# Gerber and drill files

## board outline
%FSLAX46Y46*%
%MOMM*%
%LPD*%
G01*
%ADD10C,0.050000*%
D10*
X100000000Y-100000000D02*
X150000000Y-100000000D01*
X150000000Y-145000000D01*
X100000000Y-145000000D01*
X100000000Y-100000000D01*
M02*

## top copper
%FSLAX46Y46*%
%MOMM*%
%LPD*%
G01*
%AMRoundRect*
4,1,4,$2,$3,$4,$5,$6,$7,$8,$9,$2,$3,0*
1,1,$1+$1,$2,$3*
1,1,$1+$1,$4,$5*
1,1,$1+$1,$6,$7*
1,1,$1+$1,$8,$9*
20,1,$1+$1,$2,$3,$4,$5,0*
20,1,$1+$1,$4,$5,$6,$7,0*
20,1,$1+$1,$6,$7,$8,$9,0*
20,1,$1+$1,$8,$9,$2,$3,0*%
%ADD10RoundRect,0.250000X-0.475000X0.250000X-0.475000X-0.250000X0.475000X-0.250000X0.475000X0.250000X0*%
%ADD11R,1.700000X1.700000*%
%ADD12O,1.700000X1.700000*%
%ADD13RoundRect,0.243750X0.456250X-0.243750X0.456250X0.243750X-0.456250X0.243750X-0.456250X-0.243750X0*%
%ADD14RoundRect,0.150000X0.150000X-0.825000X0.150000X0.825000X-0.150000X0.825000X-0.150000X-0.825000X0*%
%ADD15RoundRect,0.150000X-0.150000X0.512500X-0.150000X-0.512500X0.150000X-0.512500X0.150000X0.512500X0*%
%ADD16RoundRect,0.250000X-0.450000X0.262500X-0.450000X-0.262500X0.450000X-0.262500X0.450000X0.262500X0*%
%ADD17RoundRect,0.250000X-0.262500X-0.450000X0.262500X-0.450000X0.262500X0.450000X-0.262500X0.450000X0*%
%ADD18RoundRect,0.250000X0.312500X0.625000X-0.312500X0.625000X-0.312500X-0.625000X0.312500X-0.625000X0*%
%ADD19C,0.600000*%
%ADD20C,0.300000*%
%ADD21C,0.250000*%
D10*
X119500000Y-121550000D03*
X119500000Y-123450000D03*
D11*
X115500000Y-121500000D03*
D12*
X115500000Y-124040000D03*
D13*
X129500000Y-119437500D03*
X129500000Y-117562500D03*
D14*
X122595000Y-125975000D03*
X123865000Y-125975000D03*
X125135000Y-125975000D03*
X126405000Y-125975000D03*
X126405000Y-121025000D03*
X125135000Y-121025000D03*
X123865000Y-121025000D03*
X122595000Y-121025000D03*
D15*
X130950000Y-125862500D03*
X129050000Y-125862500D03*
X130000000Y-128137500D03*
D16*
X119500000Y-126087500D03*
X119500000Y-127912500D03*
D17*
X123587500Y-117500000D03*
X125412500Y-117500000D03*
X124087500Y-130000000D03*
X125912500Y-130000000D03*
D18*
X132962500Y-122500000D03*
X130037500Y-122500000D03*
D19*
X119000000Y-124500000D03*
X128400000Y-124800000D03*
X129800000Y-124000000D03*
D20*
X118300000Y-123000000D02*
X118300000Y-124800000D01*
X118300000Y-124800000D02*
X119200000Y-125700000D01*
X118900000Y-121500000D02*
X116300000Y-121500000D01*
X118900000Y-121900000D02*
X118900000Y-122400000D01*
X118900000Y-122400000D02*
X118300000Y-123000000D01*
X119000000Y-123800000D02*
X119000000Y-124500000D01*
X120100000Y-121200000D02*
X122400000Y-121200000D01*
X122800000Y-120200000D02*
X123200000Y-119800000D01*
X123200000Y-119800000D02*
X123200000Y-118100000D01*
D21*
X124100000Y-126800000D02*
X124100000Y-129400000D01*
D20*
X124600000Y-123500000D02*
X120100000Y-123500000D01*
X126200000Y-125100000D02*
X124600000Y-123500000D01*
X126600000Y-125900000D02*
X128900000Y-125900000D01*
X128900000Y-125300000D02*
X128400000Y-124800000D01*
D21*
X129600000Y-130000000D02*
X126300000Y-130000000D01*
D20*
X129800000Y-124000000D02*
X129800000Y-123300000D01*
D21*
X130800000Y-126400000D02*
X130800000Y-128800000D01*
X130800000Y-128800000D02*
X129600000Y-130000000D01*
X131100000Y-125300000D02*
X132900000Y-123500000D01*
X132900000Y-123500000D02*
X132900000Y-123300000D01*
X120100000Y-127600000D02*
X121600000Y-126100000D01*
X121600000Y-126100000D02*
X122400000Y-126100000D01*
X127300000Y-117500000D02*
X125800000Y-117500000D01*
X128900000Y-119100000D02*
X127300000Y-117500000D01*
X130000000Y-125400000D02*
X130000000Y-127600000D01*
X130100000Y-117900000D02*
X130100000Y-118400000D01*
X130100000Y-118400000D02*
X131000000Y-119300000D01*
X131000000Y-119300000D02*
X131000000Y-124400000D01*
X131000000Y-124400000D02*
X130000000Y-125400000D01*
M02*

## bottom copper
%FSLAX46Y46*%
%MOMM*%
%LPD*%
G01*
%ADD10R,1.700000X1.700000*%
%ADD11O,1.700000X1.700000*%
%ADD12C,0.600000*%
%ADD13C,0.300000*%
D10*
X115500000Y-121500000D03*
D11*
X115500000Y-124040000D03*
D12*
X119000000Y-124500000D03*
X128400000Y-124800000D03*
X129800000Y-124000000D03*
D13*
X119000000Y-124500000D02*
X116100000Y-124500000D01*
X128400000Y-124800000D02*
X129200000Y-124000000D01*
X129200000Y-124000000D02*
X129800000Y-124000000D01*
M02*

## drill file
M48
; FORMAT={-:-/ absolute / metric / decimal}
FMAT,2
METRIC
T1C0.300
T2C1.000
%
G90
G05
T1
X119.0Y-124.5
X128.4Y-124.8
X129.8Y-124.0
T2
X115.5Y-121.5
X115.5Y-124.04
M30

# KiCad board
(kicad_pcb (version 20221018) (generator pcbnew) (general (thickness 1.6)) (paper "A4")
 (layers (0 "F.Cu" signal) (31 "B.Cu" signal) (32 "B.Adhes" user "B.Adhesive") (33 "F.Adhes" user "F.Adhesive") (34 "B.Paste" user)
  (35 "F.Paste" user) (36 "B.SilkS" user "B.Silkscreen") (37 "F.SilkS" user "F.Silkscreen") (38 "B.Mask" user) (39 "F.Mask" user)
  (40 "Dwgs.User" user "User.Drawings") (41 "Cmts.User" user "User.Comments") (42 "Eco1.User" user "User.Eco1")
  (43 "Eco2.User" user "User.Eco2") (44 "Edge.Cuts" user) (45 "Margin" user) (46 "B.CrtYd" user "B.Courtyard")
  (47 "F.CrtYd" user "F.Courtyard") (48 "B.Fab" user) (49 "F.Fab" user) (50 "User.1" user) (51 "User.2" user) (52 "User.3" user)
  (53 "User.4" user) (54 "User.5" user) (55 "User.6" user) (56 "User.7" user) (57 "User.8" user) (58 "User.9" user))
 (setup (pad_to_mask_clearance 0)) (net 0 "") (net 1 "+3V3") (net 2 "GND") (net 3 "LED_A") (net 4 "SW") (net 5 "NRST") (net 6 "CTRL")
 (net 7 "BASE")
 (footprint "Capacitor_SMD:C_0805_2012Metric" (layer "F.Cu") (at 119.5 122.5 -90)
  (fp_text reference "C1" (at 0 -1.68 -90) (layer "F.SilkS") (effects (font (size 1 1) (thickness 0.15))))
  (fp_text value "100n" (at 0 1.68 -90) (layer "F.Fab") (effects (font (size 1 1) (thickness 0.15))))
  (pad "1" smd roundrect (at -0.95 0 270) (size 1 1.45) (layers "F.Cu" "F.Paste" "F.Mask") (roundrect_rratio 0.25) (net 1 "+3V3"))
  (pad "2" smd roundrect (at 0.95 0 270) (size 1 1.45) (layers "F.Cu" "F.Paste" "F.Mask") (roundrect_rratio 0.25) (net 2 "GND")))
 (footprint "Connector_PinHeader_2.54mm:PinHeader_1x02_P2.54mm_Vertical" (layer "F.Cu") (at 115.5 121.5)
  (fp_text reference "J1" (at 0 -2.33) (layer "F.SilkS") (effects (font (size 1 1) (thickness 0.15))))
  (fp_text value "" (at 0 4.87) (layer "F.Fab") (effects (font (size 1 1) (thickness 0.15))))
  (pad "1" thru_hole rect (at 0 0) (size 1.7 1.7) (drill 1) (layers "*.Cu" "*.Mask") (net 1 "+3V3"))
  (pad "2" thru_hole oval (at 0 2.54) (size 1.7 1.7) (drill 1) (layers "*.Cu" "*.Mask") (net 2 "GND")))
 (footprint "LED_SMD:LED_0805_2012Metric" (layer "F.Cu") (at 129.5 118.5 90)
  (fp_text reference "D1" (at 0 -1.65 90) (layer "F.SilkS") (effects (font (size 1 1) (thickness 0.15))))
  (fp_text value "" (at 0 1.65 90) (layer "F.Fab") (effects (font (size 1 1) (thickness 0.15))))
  (pad "1" smd roundrect (at -0.9375 0 90) (size 0.975 1.4) (layers "F.Cu" "F.Paste" "F.Mask") (roundrect_rratio 0.25) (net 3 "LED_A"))
  (pad "2" smd roundrect (at 0.9375 0 90) (size 0.975 1.4) (layers "F.Cu" "F.Paste" "F.Mask") (roundrect_rratio 0.25) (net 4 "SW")))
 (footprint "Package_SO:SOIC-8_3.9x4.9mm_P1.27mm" (layer "F.Cu") (at 124.5 123.5 90)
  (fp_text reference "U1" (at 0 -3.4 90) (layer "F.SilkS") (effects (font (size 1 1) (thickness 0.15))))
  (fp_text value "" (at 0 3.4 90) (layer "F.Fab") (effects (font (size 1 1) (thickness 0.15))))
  (pad "1" smd roundrect (at -2.475 -1.905 90) (size 1.95 0.6) (layers "F.Cu" "F.Paste" "F.Mask") (roundrect_rratio 0.25) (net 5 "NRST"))
  (pad "2" smd roundrect (at -2.475 -0.635 90) (size 1.95 0.6) (layers "F.Cu" "F.Paste" "F.Mask") (roundrect_rratio 0.25) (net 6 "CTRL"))
  (pad "3" smd roundrect (at -2.475 0.635 90) (size 1.95 0.6) (layers "F.Cu" "F.Paste" "F.Mask") (roundrect_rratio 0.25))
  (pad "4" smd roundrect (at -2.475 1.905 90) (size 1.95 0.6) (layers "F.Cu" "F.Paste" "F.Mask") (roundrect_rratio 0.25) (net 2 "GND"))
  (pad "5" smd roundrect (at 2.475 1.905 90) (size 1.95 0.6) (layers "F.Cu" "F.Paste" "F.Mask") (roundrect_rratio 0.25))
  (pad "6" smd roundrect (at 2.475 0.635 90) (size 1.95 0.6) (layers "F.Cu" "F.Paste" "F.Mask") (roundrect_rratio 0.25))
  (pad "7" smd roundrect (at 2.475 -0.635 90) (size 1.95 0.6) (layers "F.Cu" "F.Paste" "F.Mask") (roundrect_rratio 0.25))
  (pad "8" smd roundrect (at 2.475 -1.905 90) (size 1.95 0.6) (layers "F.Cu" "F.Paste" "F.Mask") (roundrect_rratio 0.25) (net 1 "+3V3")))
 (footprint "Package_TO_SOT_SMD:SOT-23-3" (layer "F.Cu") (at 130 127 -90)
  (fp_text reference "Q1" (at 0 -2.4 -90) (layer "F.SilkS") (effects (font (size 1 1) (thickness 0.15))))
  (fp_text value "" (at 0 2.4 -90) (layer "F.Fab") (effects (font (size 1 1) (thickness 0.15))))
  (pad "1" smd roundrect (at -1.1375 -0.95 270) (size 1.325 0.6) (layers "F.Cu" "F.Paste" "F.Mask") (roundrect_rratio 0.25) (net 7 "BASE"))
  (pad "2" smd roundrect (at -1.1375 0.95 270) (size 1.325 0.6) (layers "F.Cu" "F.Paste" "F.Mask") (roundrect_rratio 0.25) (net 2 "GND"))
  (pad "3" smd roundrect (at 1.1375 0 270) (size 1.325 0.6) (layers "F.Cu" "F.Paste" "F.Mask") (roundrect_rratio 0.25) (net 4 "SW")))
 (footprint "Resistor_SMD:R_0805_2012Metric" (layer "F.Cu") (at 119.5 127 -90)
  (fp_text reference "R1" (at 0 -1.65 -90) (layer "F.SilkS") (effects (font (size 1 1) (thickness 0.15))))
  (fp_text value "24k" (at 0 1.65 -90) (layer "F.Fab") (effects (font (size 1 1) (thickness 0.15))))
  (pad "1" smd roundrect (at -0.9125 0 270) (size 1.025 1.4) (layers "F.Cu" "F.Paste" "F.Mask") (roundrect_rratio 0.243902) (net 1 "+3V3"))
  (pad "2" smd roundrect (at 0.9125 0 270) (size 1.025 1.4) (layers "F.Cu" "F.Paste" "F.Mask") (roundrect_rratio 0.243902) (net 5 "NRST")))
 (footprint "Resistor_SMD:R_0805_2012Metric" (layer "F.Cu") (at 124.5 117.5)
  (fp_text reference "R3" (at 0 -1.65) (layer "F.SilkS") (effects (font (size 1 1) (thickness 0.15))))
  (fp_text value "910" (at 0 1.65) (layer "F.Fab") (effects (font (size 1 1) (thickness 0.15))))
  (pad "1" smd roundrect (at -0.9125 0) (size 1.025 1.4) (layers "F.Cu" "F.Paste" "F.Mask") (roundrect_rratio 0.243902) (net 1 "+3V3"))
  (pad "2" smd roundrect (at 0.9125 0) (size 1.025 1.4) (layers "F.Cu" "F.Paste" "F.Mask") (roundrect_rratio 0.243902) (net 3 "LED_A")))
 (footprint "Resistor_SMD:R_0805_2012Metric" (layer "F.Cu") (at 125 130)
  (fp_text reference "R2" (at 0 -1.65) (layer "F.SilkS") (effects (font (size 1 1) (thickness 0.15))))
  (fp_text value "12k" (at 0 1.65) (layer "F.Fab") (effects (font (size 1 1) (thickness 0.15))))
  (pad "1" smd roundrect (at -0.9125 0) (size 1.025 1.4) (layers "F.Cu" "F.Paste" "F.Mask") (roundrect_rratio 0.243902) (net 6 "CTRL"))
  (pad "2" smd roundrect (at 0.9125 0) (size 1.025 1.4) (layers "F.Cu" "F.Paste" "F.Mask") (roundrect_rratio 0.243902) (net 7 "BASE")))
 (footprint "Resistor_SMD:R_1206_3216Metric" (layer "F.Cu") (at 131.5 122.5 180)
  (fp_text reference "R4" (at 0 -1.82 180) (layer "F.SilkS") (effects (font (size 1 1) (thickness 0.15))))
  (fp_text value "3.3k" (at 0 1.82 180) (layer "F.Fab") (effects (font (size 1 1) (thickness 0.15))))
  (pad "1" smd roundrect (at -1.4625 0 180) (size 1.125 1.75) (layers "F.Cu" "F.Paste" "F.Mask") (roundrect_rratio 0.222222) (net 7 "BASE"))
  (pad "2" smd roundrect (at 1.4625 0 180) (size 1.125 1.75) (layers "F.Cu" "F.Paste" "F.Mask") (roundrect_rratio 0.222222) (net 2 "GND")))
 (gr_rect (start 100 100) (end 150 145) (stroke (width 0.05) (type default)) (fill none) (layer "Edge.Cuts"))
 (segment (start 118.3 123) (end 118.3 124.8) (width 0.3) (layer "F.Cu") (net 1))
 (segment (start 118.3 124.8) (end 119.2 125.7) (width 0.3) (layer "F.Cu") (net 1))
 (segment (start 118.9 121.5) (end 116.3 121.5) (width 0.3) (layer "F.Cu") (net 1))
 (segment (start 118.9 121.9) (end 118.9 122.4) (width 0.3) (layer "F.Cu") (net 1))
 (segment (start 118.9 122.4) (end 118.3 123) (width 0.3) (layer "F.Cu") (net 1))
 (segment (start 119 123.8) (end 119 124.5) (width 0.3) (layer "F.Cu") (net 2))
 (segment (start 120.1 121.2) (end 122.4 121.2) (width 0.3) (layer "F.Cu") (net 1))
 (segment (start 122.8 120.2) (end 123.2 119.8) (width 0.3) (layer "F.Cu") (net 1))
 (segment (start 123.2 119.8) (end 123.2 118.1) (width 0.3) (layer "F.Cu") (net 1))
 (segment (start 124.1 126.8) (end 124.1 129.4) (width 0.25) (layer "F.Cu") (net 6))
 (segment (start 124.6 123.5) (end 120.1 123.5) (width 0.3) (layer "F.Cu") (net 2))
 (segment (start 126.2 125.1) (end 124.6 123.5) (width 0.3) (layer "F.Cu") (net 2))
 (segment (start 126.6 125.9) (end 128.9 125.9) (width 0.3) (layer "F.Cu") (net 2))
 (segment (start 128.9 125.3) (end 128.4 124.8) (width 0.3) (layer "F.Cu") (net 2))
 (segment (start 129.6 130) (end 126.3 130) (width 0.25) (layer "F.Cu") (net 7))
 (segment (start 129.8 124) (end 129.8 123.3) (width 0.3) (layer "F.Cu") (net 2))
 (segment (start 130.8 126.4) (end 130.8 128.8) (width 0.25) (layer "F.Cu") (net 7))
 (segment (start 130.8 128.8) (end 129.6 130) (width 0.25) (layer "F.Cu") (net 7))
 (segment (start 131.1 125.3) (end 132.9 123.5) (width 0.25) (layer "F.Cu") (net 7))
 (segment (start 132.9 123.5) (end 132.9 123.3) (width 0.25) (layer "F.Cu") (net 7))
 (via (at 119 124.5) (size 0.6) (drill 0.3) (layers "F.Cu" "B.Cu") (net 2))
 (via (at 128.4 124.8) (size 0.6) (drill 0.3) (layers "F.Cu" "B.Cu") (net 2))
 (via (at 129.8 124) (size 0.6) (drill 0.3) (layers "F.Cu" "B.Cu") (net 2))
 (segment (start 119 124.5) (end 116.1 124.5) (width 0.3) (layer "B.Cu") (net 2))
 (segment (start 120.1 127.6) (end 121.6 126.1) (width 0.25) (layer "F.Cu") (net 5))
 (segment (start 121.6 126.1) (end 122.4 126.1) (width 0.25) (layer "F.Cu") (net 5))
 (segment (start 127.3 117.5) (end 125.8 117.5) (width 0.25) (layer "F.Cu") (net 3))
 (segment (start 128.4 124.8) (end 129.2 124) (width 0.3) (layer "B.Cu") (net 2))
 (segment (start 128.9 119.1) (end 127.3 117.5) (width 0.25) (layer "F.Cu") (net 3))
 (segment (start 129.2 124) (end 129.8 124) (width 0.3) (layer "B.Cu") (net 2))
 (segment (start 130 125.4) (end 130 127.6) (width 0.25) (layer "F.Cu") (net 4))
 (segment (start 130.1 117.9) (end 130.1 118.4) (width 0.25) (layer "F.Cu") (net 4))
 (segment (start 130.1 118.4) (end 131 119.3) (width 0.25) (layer "F.Cu") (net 4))
 (segment (start 131 119.3) (end 131 124.4) (width 0.25) (layer "F.Cu") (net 4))
 (segment (start 131 124.4) (end 130 125.4) (width 0.25) (layer "F.Cu") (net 4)))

